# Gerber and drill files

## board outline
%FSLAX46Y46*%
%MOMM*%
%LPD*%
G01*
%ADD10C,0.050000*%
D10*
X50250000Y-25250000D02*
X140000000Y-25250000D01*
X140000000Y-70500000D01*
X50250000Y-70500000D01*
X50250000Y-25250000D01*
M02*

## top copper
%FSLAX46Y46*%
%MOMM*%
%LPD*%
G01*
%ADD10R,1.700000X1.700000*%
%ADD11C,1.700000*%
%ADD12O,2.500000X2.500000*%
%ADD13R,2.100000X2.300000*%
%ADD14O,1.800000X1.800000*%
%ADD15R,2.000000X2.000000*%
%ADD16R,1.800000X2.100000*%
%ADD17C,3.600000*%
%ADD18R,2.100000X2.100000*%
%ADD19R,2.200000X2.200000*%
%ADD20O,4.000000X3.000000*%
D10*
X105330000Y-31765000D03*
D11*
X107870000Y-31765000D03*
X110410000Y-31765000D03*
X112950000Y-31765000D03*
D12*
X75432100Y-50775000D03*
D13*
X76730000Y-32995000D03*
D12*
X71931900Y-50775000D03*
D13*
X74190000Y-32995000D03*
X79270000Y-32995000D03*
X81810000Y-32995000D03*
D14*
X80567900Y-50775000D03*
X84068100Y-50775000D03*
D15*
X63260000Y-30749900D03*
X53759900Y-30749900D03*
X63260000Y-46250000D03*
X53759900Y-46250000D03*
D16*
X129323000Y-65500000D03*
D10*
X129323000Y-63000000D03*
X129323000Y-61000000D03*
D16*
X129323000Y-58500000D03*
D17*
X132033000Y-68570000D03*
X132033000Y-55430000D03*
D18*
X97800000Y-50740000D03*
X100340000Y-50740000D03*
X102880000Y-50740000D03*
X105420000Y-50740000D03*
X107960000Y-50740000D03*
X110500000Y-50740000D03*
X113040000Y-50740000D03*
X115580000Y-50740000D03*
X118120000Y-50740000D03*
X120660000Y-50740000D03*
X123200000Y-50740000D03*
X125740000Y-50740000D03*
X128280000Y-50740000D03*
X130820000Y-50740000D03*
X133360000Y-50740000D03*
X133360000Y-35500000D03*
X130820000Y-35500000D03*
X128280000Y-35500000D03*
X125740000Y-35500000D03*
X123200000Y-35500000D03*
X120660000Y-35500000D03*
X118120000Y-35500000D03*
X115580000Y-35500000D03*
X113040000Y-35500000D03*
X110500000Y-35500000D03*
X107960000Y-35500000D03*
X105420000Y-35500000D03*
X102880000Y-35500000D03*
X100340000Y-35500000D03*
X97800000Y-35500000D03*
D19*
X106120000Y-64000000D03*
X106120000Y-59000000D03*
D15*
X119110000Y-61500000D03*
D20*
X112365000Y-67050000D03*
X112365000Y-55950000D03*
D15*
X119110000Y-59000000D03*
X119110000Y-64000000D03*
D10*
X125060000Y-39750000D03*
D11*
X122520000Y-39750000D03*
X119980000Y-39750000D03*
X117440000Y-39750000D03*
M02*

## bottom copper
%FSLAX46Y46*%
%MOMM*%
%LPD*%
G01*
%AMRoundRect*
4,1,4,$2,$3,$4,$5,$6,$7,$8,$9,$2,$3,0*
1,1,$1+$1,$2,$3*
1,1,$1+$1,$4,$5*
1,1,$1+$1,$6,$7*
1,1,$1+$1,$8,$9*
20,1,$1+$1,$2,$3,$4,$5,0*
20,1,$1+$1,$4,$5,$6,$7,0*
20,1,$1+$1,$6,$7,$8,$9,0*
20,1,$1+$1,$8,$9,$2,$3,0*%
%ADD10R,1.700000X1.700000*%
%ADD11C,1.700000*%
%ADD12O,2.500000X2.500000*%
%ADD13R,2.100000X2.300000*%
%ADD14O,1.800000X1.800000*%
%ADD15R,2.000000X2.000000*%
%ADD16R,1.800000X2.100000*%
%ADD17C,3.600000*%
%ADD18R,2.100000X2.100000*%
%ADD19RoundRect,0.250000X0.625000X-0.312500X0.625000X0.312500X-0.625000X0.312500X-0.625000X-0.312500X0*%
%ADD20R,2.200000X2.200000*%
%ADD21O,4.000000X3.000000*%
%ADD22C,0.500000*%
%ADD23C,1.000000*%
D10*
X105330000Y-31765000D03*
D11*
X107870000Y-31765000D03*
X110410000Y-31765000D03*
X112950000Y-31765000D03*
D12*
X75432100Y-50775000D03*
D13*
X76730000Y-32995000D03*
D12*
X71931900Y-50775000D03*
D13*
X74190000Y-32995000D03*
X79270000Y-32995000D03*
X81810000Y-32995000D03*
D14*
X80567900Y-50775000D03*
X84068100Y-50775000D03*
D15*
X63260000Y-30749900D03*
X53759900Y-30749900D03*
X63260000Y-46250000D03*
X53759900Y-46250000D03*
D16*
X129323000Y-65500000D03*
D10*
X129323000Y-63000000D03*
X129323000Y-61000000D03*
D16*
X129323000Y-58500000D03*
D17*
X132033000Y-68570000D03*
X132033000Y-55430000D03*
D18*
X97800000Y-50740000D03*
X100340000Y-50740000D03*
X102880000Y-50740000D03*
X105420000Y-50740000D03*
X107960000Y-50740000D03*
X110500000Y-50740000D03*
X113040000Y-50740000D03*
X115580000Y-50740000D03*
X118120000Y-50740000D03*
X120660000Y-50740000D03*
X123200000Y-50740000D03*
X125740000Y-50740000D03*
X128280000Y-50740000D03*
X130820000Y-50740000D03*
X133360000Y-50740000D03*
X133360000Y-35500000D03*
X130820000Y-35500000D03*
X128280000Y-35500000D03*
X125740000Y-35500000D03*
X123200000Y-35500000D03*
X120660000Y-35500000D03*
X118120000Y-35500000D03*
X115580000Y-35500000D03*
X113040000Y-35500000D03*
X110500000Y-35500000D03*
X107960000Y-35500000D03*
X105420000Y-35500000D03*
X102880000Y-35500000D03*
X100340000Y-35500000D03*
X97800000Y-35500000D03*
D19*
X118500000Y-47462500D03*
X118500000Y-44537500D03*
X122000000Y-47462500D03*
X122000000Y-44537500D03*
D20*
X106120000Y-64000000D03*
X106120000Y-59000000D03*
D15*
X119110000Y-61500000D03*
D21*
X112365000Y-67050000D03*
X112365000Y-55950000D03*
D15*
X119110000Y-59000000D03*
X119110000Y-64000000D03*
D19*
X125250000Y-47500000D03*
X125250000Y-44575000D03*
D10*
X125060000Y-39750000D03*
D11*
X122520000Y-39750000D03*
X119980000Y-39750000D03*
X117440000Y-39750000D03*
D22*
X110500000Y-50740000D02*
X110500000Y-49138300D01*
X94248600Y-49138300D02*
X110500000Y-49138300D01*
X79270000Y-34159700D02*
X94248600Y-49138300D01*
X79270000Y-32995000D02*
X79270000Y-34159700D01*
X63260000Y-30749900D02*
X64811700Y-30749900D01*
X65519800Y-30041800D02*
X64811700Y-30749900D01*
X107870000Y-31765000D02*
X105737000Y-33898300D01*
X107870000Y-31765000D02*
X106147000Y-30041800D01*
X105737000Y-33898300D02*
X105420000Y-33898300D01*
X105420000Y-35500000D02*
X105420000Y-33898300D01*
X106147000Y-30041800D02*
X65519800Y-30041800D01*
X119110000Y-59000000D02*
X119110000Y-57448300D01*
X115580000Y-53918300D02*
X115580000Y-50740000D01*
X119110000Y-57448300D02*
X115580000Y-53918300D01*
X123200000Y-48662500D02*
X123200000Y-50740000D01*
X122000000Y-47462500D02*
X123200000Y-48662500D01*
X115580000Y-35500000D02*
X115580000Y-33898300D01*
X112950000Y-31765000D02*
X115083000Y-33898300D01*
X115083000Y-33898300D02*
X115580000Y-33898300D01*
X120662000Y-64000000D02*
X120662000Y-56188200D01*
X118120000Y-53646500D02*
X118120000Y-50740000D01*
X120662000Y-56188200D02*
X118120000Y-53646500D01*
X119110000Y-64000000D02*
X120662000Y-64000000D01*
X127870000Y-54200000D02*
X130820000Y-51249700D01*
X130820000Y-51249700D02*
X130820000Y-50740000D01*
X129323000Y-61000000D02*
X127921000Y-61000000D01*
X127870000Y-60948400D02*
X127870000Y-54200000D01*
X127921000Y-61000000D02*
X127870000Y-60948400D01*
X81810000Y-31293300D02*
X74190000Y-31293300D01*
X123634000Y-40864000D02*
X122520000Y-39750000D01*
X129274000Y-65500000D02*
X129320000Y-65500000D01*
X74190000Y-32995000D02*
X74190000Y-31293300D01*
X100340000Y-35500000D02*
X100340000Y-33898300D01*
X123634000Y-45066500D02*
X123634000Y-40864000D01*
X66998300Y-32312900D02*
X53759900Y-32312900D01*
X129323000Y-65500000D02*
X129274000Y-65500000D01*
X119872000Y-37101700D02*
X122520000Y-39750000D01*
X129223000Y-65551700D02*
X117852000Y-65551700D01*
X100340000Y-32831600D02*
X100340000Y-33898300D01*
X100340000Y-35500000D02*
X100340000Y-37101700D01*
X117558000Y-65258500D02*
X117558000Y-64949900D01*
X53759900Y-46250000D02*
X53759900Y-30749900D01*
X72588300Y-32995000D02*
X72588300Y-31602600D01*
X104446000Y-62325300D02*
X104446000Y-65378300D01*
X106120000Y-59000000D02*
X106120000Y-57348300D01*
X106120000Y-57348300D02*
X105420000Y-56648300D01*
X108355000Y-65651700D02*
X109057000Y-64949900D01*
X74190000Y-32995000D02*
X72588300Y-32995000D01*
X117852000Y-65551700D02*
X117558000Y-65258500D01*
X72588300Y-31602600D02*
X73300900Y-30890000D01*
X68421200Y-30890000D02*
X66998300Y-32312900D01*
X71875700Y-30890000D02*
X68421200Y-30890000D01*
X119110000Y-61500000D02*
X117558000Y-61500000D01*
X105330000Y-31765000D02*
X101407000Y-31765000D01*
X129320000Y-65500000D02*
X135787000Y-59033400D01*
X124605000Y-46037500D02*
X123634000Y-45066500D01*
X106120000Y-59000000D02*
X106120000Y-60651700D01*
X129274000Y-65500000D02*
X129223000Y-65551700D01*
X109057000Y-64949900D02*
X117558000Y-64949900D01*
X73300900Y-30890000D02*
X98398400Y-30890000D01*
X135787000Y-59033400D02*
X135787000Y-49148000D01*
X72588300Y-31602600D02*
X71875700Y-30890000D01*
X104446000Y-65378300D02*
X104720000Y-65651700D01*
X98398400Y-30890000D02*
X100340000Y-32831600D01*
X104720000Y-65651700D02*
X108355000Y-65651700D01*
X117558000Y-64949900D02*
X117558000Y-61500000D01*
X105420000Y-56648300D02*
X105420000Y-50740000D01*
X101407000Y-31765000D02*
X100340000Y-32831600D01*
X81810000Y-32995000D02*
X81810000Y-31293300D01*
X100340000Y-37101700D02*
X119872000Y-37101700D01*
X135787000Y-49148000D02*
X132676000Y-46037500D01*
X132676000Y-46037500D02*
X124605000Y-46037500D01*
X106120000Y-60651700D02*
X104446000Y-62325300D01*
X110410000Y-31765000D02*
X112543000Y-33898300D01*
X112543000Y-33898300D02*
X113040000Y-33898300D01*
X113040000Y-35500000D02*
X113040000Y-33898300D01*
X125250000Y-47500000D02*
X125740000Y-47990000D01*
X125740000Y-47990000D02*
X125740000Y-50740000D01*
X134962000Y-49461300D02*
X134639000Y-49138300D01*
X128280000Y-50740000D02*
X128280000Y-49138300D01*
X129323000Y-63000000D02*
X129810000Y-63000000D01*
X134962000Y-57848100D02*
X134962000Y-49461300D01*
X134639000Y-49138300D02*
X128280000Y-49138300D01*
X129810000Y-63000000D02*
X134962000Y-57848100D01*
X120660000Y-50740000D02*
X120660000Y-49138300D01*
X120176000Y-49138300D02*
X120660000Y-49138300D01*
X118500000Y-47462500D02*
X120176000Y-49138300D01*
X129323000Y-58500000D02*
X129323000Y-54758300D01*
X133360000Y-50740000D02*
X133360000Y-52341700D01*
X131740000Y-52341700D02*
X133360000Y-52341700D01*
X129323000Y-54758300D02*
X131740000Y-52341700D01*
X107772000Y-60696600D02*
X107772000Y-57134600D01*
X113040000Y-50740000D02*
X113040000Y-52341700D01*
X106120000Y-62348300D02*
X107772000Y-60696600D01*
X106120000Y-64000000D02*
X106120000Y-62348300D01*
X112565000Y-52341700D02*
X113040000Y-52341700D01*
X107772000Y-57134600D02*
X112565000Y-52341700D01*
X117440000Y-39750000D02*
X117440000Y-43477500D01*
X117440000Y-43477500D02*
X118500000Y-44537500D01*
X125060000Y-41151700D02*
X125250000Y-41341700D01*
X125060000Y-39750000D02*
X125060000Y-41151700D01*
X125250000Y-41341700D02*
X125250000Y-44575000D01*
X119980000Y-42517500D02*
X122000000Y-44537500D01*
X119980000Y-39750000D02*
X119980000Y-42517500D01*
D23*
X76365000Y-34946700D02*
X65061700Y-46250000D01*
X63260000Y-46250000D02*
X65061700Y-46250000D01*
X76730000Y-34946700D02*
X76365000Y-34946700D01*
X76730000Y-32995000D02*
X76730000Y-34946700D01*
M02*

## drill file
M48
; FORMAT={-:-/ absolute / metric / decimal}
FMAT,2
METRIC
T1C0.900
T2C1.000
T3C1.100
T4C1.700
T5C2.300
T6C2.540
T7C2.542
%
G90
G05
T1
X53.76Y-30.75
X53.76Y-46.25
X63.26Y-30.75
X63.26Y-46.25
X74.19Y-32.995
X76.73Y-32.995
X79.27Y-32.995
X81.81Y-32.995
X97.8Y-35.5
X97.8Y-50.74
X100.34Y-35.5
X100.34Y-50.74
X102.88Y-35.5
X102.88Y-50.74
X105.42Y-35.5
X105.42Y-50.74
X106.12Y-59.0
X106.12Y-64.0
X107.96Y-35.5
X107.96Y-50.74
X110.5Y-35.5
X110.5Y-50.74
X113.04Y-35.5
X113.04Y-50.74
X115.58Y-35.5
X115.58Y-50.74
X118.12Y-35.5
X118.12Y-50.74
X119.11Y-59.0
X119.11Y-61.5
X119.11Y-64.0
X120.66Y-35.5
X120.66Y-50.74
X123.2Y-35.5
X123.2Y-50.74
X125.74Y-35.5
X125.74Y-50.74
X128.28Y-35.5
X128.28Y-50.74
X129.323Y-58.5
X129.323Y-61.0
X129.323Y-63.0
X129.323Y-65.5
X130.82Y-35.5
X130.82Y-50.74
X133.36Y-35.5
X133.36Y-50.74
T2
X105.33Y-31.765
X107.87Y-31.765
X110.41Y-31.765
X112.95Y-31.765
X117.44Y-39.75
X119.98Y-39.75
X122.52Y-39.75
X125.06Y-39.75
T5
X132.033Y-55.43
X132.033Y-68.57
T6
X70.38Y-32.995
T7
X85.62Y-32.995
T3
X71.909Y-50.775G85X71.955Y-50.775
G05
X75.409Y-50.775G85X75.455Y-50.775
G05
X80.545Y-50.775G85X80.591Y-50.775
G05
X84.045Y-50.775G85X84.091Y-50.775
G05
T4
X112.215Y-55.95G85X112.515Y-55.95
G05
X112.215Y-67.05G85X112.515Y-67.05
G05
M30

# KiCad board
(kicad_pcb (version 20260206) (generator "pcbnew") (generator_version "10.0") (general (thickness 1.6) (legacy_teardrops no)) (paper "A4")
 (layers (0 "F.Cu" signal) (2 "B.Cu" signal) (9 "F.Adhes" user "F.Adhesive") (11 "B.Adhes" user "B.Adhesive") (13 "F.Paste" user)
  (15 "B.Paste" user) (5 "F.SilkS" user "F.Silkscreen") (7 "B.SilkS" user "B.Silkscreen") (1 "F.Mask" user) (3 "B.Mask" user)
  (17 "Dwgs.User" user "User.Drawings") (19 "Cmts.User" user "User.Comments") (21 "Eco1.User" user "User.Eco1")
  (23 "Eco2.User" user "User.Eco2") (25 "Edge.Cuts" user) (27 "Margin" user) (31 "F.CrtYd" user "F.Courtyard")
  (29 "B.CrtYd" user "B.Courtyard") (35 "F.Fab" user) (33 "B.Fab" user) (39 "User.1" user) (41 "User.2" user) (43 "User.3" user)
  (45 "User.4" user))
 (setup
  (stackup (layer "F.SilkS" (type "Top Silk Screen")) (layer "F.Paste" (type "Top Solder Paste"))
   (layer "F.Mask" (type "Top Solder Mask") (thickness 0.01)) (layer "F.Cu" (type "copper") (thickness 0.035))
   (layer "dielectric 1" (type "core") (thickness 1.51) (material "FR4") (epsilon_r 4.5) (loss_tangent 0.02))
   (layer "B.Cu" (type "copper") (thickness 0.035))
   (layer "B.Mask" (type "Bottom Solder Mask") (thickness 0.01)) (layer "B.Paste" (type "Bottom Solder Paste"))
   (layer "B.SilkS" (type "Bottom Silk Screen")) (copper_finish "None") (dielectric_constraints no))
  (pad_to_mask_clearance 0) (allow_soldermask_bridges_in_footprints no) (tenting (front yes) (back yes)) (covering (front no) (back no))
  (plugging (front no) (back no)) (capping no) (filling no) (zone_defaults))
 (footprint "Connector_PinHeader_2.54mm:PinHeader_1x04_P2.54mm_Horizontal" (layer "F.Cu") (at 105.33 31.765 90)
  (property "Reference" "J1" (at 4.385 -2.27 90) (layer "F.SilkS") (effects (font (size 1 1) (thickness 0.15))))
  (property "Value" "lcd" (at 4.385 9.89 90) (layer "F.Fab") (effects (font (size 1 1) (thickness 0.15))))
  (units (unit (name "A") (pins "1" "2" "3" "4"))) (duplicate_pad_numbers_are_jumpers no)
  (pad "1" thru_hole rect (at 0 0 90) (size 1.7 1.7) (drill 1) (layers "*.Cu" "*.Mask") (remove_unused_layers no) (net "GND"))
  (pad "2" thru_hole circle (at 0 2.54 90) (size 1.7 1.7) (drill 1) (layers "*.Cu" "*.Mask") (remove_unused_layers no) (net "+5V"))
  (pad "3" thru_hole circle (at 0 5.08 90) (size 1.7 1.7) (drill 1) (layers "*.Cu" "*.Mask") (remove_unused_layers no) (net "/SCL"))
  (pad "4" thru_hole circle (at 0 7.62 90) (size 1.7 1.7) (drill 1) (layers "*.Cu" "*.Mask") (remove_unused_layers no) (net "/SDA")))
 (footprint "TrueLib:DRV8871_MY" (layer "F.Cu") (at 78 41.885)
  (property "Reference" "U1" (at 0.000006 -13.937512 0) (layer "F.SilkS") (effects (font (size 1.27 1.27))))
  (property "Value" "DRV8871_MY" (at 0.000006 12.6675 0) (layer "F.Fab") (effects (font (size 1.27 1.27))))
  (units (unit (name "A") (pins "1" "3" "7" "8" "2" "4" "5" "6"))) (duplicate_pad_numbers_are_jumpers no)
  (pad "" np_thru_hole circle (at -7.62 -8.89) (size 2.54 2.54) (drill 2.54) (layers "*.Cu" "*.Mask"))
  (pad "" np_thru_hole circle (at 7.62 -8.89) (size 2.542 2.542) (drill 2.542) (layers "*.Cu" "*.Mask"))
  (pad "1" thru_hole oval (at -2.5679 8.89) (size 2.5 2.5) (drill oval 1.1457 1.1) (layers "*.Cu" "*.Mask") (remove_unused_layers no)
   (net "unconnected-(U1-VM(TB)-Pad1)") (solder_mask_margin 0.1016) (solder_paste_margin 0) (thermal_bridge_angle 0))
  (pad "2" thru_hole rect (at -1.27 -8.89) (size 2.1 2.3) (drill 0.9) (layers "*.Cu" "*.Mask") (remove_unused_layers no) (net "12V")
   (solder_mask_margin 0.102) (solder_paste_margin 0) (thermal_bridge_angle 0))
  (pad "3" thru_hole oval (at -6.0681 8.89) (size 2.5 2.5) (drill oval 1.1457 1.1) (layers "*.Cu" "*.Mask") (remove_unused_layers no)
   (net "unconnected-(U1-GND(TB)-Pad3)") (solder_mask_margin 0.1016) (solder_paste_margin 0) (thermal_bridge_angle 0))
  (pad "4" thru_hole rect (at -3.81 -8.89) (size 2.1 2.3) (drill 0.9) (layers "*.Cu" "*.Mask") (remove_unused_layers no) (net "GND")
   (solder_mask_margin 0.102) (solder_paste_margin 0) (thermal_bridge_angle 0))
  (pad "5" thru_hole rect (at 1.27 -8.89) (size 2.1 2.3) (drill 0.9) (layers "*.Cu" "*.Mask") (remove_unused_layers no) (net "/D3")
   (solder_mask_margin 0.102) (solder_paste_margin 0) (thermal_bridge_angle 0))
  (pad "6" thru_hole rect (at 3.81 -8.89) (size 2.1 2.3) (drill 0.9) (layers "*.Cu" "*.Mask") (remove_unused_layers no) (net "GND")
   (solder_mask_margin 0.102) (solder_paste_margin 0) (thermal_bridge_angle 0))
  (pad "7" thru_hole oval (at 2.5679 8.89) (size 1.8 1.8) (drill oval 1.1457 1.1) (layers "*.Cu" "*.Mask") (remove_unused_layers no)
   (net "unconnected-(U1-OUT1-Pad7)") (solder_mask_margin 0.1016) (solder_paste_margin 0) (thermal_bridge_angle 0))
  (pad "8" thru_hole oval (at 6.0681 8.89) (size 1.8 1.8) (drill oval 1.1457 1.1) (layers "*.Cu" "*.Mask") (remove_unused_layers no)
   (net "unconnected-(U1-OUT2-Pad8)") (solder_mask_margin 0.1016) (solder_paste_margin 0) (thermal_bridge_angle 0)))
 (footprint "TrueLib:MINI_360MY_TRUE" (layer "F.Cu") (at 63.26 46.25 90)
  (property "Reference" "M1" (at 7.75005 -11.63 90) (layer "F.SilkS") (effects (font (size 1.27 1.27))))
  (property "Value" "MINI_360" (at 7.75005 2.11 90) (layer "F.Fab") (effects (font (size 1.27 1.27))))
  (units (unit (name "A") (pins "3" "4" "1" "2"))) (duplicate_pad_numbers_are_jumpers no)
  (pad "1" thru_hole rect (at 15.5001 0 90) (size 2 2) (drill 0.9) (layers "*.Cu" "*.Mask") (remove_unused_layers no) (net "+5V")
   (solder_mask_margin 0.1) (solder_paste_margin 0) (thermal_bridge_angle 0))
  (pad "2" thru_hole rect (at 15.5001 -9.5001 90) (size 2 2) (drill 0.9) (layers "*.Cu" "*.Mask") (remove_unused_layers no) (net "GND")
   (solder_mask_margin 0.1) (solder_paste_margin 0) (thermal_bridge_angle 0))
  (pad "3" thru_hole rect (at 0 0 90) (size 2 2) (drill 0.9) (layers "*.Cu" "*.Mask") (remove_unused_layers no) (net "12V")
   (solder_mask_margin 0.1) (solder_paste_margin 0) (thermal_bridge_angle 0))
  (pad "4" thru_hole rect (at 0 -9.5001 90) (size 2 2) (drill 0.9) (layers "*.Cu" "*.Mask") (remove_unused_layers no) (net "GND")
   (solder_mask_margin 0.1) (solder_paste_margin 0) (thermal_bridge_angle 0)))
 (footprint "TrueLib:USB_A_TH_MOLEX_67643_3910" (layer "F.Cu") (at 129.323 65.5 90)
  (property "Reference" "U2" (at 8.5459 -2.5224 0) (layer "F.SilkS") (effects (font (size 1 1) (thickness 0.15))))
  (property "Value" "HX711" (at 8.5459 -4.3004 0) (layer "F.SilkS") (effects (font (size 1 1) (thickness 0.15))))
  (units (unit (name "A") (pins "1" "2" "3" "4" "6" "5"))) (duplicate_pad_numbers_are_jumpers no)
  (pad "1" thru_hole rect (at 0 0 90) (size 2.1 1.8) (drill 0.9) (layers "*.Cu" "*.Mask") (remove_unused_layers no) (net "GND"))
  (pad "2" thru_hole rect (at 2.5 0 90) (size 1.7 1.7) (drill 0.9) (layers "*.Cu" "*.Mask") (remove_unused_layers no) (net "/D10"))
  (pad "3" thru_hole rect (at 4.5 0 90) (size 1.7 1.7) (drill 0.9) (layers "*.Cu" "*.Mask") (remove_unused_layers no) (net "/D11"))
  (pad "4" thru_hole rect (at 7 0 90) (size 2.1 1.8) (drill 0.9) (layers "*.Cu" "*.Mask") (remove_unused_layers no) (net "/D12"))
  (pad "5" thru_hole circle (at -3.07 2.71 90) (size 3.6 3.6) (drill 2.3) (layers "*.Cu" "*.Mask") (remove_unused_layers no)
   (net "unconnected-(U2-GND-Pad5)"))
  (pad "6" thru_hole circle (at 10.07 2.71 90) (size 3.6 3.6) (drill 2.3) (layers "*.Cu" "*.Mask") (remove_unused_layers no)
   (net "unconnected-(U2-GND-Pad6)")))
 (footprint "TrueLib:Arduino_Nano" (layer "F.Cu") (at 97.8 50.74 90)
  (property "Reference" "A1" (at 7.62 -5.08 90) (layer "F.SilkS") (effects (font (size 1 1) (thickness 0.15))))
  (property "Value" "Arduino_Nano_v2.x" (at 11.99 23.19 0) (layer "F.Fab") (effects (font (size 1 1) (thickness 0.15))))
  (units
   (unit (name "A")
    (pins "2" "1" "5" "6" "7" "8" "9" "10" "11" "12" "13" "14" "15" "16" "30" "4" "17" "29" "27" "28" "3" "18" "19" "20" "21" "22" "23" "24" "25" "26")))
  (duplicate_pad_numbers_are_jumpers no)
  (pad "1" thru_hole rect (at 0 0 90) (size 2.1 2.1) (drill 0.9) (layers "*.Cu" "*.Mask") (remove_unused_layers no)
   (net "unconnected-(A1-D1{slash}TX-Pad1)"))
  (pad "2" thru_hole rect (at 0 2.54 90) (size 2.1 2.1) (drill 0.9) (layers "*.Cu" "*.Mask") (remove_unused_layers no)
   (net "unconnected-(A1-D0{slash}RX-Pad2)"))
  (pad "3" thru_hole rect (at 0 5.08 90) (size 2.1 2.1) (drill 0.9) (layers "*.Cu" "*.Mask") (remove_unused_layers no)
   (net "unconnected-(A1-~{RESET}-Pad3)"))
  (pad "4" thru_hole rect (at 0 7.62 90) (size 2.1 2.1) (drill 0.9) (layers "*.Cu" "*.Mask") (remove_unused_layers no) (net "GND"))
  (pad "5" thru_hole rect (at 0 10.16 90) (size 2.1 2.1) (drill 0.9) (layers "*.Cu" "*.Mask") (remove_unused_layers no)
   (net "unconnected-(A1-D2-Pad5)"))
  (pad "6" thru_hole rect (at 0 12.7 90) (size 2.1 2.1) (drill 0.9) (layers "*.Cu" "*.Mask") (remove_unused_layers no) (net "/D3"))
  (pad "7" thru_hole rect (at 0 15.24 90) (size 2.1 2.1) (drill 0.9) (layers "*.Cu" "*.Mask") (remove_unused_layers no) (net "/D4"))
  (pad "8" thru_hole rect (at 0 17.78 90) (size 2.1 2.1) (drill 0.9) (layers "*.Cu" "*.Mask") (remove_unused_layers no) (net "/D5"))
  (pad "9" thru_hole rect (at 0 20.32 90) (size 2.1 2.1) (drill 0.9) (layers "*.Cu" "*.Mask") (remove_unused_layers no) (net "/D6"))
  (pad "10" thru_hole rect (at 0 22.86 90) (size 2.1 2.1) (drill 0.9) (layers "*.Cu" "*.Mask") (remove_unused_layers no) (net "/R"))
  (pad "11" thru_hole rect (at 0 25.4 90) (size 2.1 2.1) (drill 0.9) (layers "*.Cu" "*.Mask") (remove_unused_layers no) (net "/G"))
  (pad "12" thru_hole rect (at 0 27.94 90) (size 2.1 2.1) (drill 0.9) (layers "*.Cu" "*.Mask") (remove_unused_layers no) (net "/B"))
  (pad "13" thru_hole rect (at 0 30.48 90) (size 2.1 2.1) (drill 0.9) (layers "*.Cu" "*.Mask") (remove_unused_layers no) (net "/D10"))
  (pad "14" thru_hole rect (at 0 33.02 90) (size 2.1 2.1) (drill 0.9) (layers "*.Cu" "*.Mask") (remove_unused_layers no) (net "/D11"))
  (pad "15" thru_hole rect (at 0 35.56 90) (size 2.1 2.1) (drill 0.9) (layers "*.Cu" "*.Mask") (remove_unused_layers no) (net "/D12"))
  (pad "16" thru_hole rect (at 15.24 35.56 90) (size 2.1 2.1) (drill 0.9) (layers "*.Cu" "*.Mask") (remove_unused_layers no)
   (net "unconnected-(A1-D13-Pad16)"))
  (pad "17" thru_hole rect (at 15.24 33.02 90) (size 2.1 2.1) (drill 0.9) (layers "*.Cu" "*.Mask") (remove_unused_layers no)
   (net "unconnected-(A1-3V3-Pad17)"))
  (pad "18" thru_hole rect (at 15.24 30.48 90) (size 2.1 2.1) (drill 0.9) (layers "*.Cu" "*.Mask") (remove_unused_layers no)
   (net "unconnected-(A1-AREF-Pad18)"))
  (pad "19" thru_hole rect (at 15.24 27.94 90) (size 2.1 2.1) (drill 0.9) (layers "*.Cu" "*.Mask") (remove_unused_layers no)
   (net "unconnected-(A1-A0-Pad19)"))
  (pad "20" thru_hole rect (at 15.24 25.4 90) (size 2.1 2.1) (drill 0.9) (layers "*.Cu" "*.Mask") (remove_unused_layers no)
   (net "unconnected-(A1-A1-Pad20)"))
  (pad "21" thru_hole rect (at 15.24 22.86 90) (size 2.1 2.1) (drill 0.9) (layers "*.Cu" "*.Mask") (remove_unused_layers no)
   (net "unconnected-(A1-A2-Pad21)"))
  (pad "22" thru_hole rect (at 15.24 20.32 90) (size 2.1 2.1) (drill 0.9) (layers "*.Cu" "*.Mask") (remove_unused_layers no)
   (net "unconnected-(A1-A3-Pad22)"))
  (pad "23" thru_hole rect (at 15.24 17.78 90) (size 2.1 2.1) (drill 0.9) (layers "*.Cu" "*.Mask") (remove_unused_layers no) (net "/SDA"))
  (pad "24" thru_hole rect (at 15.24 15.24 90) (size 2.1 2.1) (drill 0.9) (layers "*.Cu" "*.Mask") (remove_unused_layers no) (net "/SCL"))
  (pad "25" thru_hole rect (at 15.24 12.7 90) (size 2.1 2.1) (drill 0.9) (layers "*.Cu" "*.Mask") (remove_unused_layers no)
   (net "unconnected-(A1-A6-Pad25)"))
  (pad "26" thru_hole rect (at 15.24 10.16 90) (size 2.1 2.1) (drill 0.9) (layers "*.Cu" "*.Mask") (remove_unused_layers no)
   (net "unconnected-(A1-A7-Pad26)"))
  (pad "27" thru_hole rect (at 15.24 7.62 90) (size 2.1 2.1) (drill 0.9) (layers "*.Cu" "*.Mask") (remove_unused_layers no) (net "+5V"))
  (pad "28" thru_hole rect (at 15.24 5.08 90) (size 2.1 2.1) (drill 0.9) (layers "*.Cu" "*.Mask") (remove_unused_layers no)
   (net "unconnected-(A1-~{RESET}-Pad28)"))
  (pad "29" thru_hole rect (at 15.24 2.54 90) (size 2.1 2.1) (drill 0.9) (layers "*.Cu" "*.Mask") (remove_unused_layers no) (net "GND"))
  (pad "30" thru_hole rect (at 15.24 0 90) (size 2.1 2.1) (drill 0.9) (layers "*.Cu" "*.Mask") (remove_unused_layers no)
   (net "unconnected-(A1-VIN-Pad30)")))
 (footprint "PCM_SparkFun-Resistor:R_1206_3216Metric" (layer "B.Cu") (at 118.5 46 90)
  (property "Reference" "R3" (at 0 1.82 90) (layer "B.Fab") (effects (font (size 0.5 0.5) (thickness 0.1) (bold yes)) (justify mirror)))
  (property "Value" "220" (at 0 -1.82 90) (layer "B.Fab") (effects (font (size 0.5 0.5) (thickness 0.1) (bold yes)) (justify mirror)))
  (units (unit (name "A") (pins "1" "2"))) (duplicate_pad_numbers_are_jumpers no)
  (pad "1" smd roundrect (at -1.4625 0 90) (size 1.125 1.75) (layers "B.Cu" "B.Mask" "B.Paste") (roundrect_rratio 0.222222) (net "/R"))
  (pad "2" smd roundrect (at 1.4625 0 90) (size 1.125 1.75) (layers "B.Cu" "B.Mask" "B.Paste") (roundrect_rratio 0.222222)
   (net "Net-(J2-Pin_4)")))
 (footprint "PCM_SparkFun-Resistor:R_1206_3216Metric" (layer "B.Cu") (at 122 46 90)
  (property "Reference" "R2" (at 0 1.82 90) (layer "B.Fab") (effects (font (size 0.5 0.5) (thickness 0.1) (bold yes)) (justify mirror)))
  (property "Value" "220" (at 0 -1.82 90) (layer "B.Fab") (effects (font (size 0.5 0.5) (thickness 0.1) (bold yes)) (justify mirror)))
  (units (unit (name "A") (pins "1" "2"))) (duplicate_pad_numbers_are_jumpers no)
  (pad "1" smd roundrect (at -1.4625 0 90) (size 1.125 1.75) (layers "B.Cu" "B.Mask" "B.Paste") (roundrect_rratio 0.222222) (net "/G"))
  (pad "2" smd roundrect (at 1.4625 0 90) (size 1.125 1.75) (layers "B.Cu" "B.Mask" "B.Paste") (roundrect_rratio 0.222222)
   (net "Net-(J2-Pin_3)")))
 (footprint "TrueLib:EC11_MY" (layer "B.Cu") (at 112.115 61.5 90)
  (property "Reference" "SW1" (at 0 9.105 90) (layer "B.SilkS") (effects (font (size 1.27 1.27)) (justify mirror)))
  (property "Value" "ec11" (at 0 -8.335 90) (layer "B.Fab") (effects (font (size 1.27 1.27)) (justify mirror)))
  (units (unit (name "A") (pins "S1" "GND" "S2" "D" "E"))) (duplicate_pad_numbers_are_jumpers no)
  (pad "D" thru_hole rect (at -2.5 -5.995 90) (size 2.2 2.2) (drill 0.9) (layers "*.Cu" "*.Mask") (remove_unused_layers no) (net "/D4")
   (solder_mask_margin 0.05) (solder_paste_margin 0) (thermal_bridge_angle 0))
  (pad "E" thru_hole rect (at 2.5 -5.995 90) (size 2.2 2.2) (drill 0.9) (layers "*.Cu" "*.Mask") (remove_unused_layers no) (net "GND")
   (solder_mask_margin 0.05) (solder_paste_margin 0) (thermal_bridge_angle 0))
  (pad "GND" thru_hole rect (at 0 6.995 90) (size 2 2) (drill 0.9) (layers "*.Cu" "*.Mask") (remove_unused_layers no) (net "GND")
   (solder_mask_margin 0.05) (solder_paste_margin 0) (thermal_bridge_angle 0))
  (pad "MP1" thru_hole oval (at -5.55 0.25 90) (size 3 4) (drill oval 1.7 2) (layers "*.Cu" "*.Mask") (remove_unused_layers no)
   (solder_mask_margin 0.05) (solder_paste_margin 0) (thermal_bridge_angle 0))
  (pad "MP2" thru_hole oval (at 5.55 0.25 90) (size 3 4) (drill oval 1.7 2) (layers "*.Cu" "*.Mask") (remove_unused_layers no)
   (solder_mask_margin 0.05) (solder_paste_margin 0) (thermal_bridge_angle 0))
  (pad "S1" thru_hole rect (at 2.5 6.995 90) (size 2 2) (drill 0.9) (layers "*.Cu" "*.Mask") (remove_unused_layers no) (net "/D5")
   (solder_mask_margin 0.05) (solder_paste_margin 0) (thermal_bridge_angle 0))
  (pad "S2" thru_hole rect (at -2.5 6.995 90) (size 2 2) (drill 0.9) (layers "*.Cu" "*.Mask") (remove_unused_layers no) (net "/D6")
   (solder_mask_margin 0.05) (solder_paste_margin 0) (thermal_bridge_angle 0))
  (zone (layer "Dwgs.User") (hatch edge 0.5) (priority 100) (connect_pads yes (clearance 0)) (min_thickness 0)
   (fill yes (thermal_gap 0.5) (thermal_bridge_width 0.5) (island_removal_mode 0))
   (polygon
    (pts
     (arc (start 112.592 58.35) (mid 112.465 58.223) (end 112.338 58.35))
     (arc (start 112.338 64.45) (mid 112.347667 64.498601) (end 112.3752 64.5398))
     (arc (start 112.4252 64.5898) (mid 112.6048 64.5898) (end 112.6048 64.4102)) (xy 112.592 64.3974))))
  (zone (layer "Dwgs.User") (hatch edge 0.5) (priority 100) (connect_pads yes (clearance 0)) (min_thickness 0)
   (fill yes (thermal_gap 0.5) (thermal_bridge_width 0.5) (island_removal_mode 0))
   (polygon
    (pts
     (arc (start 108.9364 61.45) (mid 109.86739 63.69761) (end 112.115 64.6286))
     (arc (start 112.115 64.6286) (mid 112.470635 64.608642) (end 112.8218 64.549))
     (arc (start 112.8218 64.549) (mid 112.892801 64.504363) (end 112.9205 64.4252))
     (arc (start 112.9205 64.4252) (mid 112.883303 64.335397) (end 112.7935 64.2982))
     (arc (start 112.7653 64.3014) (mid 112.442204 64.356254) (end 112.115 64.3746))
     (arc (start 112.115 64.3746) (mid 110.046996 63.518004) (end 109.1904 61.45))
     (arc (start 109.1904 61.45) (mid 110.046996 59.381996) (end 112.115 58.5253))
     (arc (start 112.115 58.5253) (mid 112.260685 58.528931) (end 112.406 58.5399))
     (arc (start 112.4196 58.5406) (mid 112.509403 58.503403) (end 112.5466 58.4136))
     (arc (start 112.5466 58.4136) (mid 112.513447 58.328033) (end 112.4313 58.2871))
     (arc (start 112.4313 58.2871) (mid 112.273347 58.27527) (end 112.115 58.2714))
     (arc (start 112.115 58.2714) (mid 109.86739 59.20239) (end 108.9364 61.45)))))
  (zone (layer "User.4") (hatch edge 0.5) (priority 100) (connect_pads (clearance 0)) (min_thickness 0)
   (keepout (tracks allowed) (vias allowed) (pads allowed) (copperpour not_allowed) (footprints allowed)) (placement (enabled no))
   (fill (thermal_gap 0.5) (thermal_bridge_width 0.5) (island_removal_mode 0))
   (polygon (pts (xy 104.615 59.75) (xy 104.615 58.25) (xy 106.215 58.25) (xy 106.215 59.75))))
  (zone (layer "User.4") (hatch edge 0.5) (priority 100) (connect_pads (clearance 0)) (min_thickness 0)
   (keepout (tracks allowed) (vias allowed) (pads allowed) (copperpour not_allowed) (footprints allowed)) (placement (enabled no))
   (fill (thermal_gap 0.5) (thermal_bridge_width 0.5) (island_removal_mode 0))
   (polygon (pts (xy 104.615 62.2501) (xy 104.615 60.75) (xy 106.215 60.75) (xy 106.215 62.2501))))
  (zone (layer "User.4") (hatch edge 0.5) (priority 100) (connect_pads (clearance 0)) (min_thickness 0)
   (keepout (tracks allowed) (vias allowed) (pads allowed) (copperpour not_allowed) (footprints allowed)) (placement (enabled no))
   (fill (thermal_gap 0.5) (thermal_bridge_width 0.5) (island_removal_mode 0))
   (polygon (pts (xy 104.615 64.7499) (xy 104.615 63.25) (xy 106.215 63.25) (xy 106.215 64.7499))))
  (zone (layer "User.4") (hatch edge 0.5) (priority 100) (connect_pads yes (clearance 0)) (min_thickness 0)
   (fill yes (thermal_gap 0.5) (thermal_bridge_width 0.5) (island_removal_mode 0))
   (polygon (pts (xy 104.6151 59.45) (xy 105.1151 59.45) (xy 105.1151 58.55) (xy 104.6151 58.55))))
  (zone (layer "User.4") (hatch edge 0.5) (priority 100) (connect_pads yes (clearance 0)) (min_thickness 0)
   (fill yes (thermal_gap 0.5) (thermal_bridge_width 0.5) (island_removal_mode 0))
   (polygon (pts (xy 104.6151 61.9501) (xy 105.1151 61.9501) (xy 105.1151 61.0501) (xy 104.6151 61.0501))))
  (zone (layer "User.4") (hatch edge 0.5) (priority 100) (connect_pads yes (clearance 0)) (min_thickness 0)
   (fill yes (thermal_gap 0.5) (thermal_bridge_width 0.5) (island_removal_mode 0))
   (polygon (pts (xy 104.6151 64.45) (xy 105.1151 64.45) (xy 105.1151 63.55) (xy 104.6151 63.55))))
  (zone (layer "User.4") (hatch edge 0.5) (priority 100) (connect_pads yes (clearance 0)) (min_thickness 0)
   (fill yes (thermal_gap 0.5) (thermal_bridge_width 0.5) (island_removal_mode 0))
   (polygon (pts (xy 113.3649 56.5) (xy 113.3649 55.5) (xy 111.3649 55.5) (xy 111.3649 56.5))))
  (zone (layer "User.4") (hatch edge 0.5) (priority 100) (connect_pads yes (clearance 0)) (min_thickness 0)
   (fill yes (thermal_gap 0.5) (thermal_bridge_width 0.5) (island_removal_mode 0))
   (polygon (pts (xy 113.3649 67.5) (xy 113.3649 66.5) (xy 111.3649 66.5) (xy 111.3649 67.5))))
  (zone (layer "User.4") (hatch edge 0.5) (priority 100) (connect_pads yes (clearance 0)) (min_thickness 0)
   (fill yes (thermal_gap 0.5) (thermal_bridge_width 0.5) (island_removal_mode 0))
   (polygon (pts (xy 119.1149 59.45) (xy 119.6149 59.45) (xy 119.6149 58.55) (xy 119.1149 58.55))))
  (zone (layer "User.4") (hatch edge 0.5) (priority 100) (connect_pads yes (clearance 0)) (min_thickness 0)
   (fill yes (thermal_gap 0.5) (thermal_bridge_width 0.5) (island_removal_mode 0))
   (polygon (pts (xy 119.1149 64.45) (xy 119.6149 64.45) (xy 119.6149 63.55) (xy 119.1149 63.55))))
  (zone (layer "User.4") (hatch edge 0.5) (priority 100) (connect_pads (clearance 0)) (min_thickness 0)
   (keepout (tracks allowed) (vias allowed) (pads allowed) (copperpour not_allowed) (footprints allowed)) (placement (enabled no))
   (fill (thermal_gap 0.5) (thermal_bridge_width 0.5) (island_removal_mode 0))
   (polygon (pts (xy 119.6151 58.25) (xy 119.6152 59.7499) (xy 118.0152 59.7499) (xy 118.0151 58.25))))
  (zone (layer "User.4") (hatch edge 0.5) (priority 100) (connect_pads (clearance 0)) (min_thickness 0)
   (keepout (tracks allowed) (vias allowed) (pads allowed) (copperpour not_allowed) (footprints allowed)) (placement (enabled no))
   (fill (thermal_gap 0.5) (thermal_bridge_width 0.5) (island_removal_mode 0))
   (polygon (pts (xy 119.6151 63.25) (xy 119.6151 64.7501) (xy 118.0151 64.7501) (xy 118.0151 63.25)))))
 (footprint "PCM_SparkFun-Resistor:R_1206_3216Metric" (layer "B.Cu") (at 125.25 46.0375 90)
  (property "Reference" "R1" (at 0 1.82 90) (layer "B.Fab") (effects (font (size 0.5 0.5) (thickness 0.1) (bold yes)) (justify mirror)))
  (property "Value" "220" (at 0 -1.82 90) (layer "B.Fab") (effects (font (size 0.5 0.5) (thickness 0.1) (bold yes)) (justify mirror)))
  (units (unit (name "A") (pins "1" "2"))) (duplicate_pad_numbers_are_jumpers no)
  (pad "1" smd roundrect (at -1.4625 0 90) (size 1.125 1.75) (layers "B.Cu" "B.Mask" "B.Paste") (roundrect_rratio 0.222222) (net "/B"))
  (pad "2" smd roundrect (at 1.4625 0 90) (size 1.125 1.75) (layers "B.Cu" "B.Mask" "B.Paste") (roundrect_rratio 0.222222)
   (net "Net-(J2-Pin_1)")))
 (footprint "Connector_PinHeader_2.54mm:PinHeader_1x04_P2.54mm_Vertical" (layer "B.Cu") (at 125.06 39.75 90)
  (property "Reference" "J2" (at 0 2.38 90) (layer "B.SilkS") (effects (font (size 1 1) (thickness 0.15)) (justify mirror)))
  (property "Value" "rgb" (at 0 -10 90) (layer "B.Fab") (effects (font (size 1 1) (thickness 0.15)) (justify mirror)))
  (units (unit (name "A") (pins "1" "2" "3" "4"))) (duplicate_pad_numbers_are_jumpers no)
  (pad "1" thru_hole rect (at 0 0 90) (size 1.7 1.7) (drill 1) (layers "*.Cu" "*.Mask") (remove_unused_layers no) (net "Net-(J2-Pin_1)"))
  (pad "2" thru_hole circle (at 0 -2.54 90) (size 1.7 1.7) (drill 1) (layers "*.Cu" "*.Mask") (remove_unused_layers no) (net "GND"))
  (pad "3" thru_hole circle (at 0 -5.08 90) (size 1.7 1.7) (drill 1) (layers "*.Cu" "*.Mask") (remove_unused_layers no)
   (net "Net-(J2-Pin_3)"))
  (pad "4" thru_hole circle (at 0 -7.62 90) (size 1.7 1.7) (drill 1) (layers "*.Cu" "*.Mask") (remove_unused_layers no)
   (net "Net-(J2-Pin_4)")))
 (gr_rect (start 50.25 25.25) (end 140 70.5) (stroke (width 0.05) (type default)) (fill no) (layer "Edge.Cuts"))
 (segment (start 110.5 50.74) (end 110.5 49.1383) (width 0.5) (layer "B.Cu") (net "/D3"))
 (segment (start 94.2486 49.1383) (end 110.5 49.1383) (width 0.5) (layer "B.Cu") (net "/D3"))
 (segment (start 79.27 34.1597) (end 94.2486 49.1383) (width 0.5) (layer "B.Cu") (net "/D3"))
 (segment (start 79.27 32.995) (end 79.27 34.1597) (width 0.5) (layer "B.Cu") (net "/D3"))
 (segment (start 63.26 30.7499) (end 64.8117 30.7499) (width 0.5) (layer "B.Cu") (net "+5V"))
 (segment (start 65.5198 30.0418) (end 64.8117 30.7499) (width 0.5) (layer "B.Cu") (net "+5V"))
 (segment (start 107.87 31.765) (end 105.737 33.8983) (width 0.5) (layer "B.Cu") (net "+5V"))
 (segment (start 107.87 31.765) (end 106.147 30.0418) (width 0.5) (layer "B.Cu") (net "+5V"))
 (segment (start 105.737 33.8983) (end 105.42 33.8983) (width 0.5) (layer "B.Cu") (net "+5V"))
 (segment (start 105.42 35.5) (end 105.42 33.8983) (width 0.5) (layer "B.Cu") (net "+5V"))
 (segment (start 106.147 30.0418) (end 65.5198 30.0418) (width 0.5) (layer "B.Cu") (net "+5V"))
 (segment (start 119.11 59) (end 119.11 57.4483) (width 0.5) (layer "B.Cu") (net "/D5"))
 (segment (start 115.58 53.9183) (end 115.58 50.74) (width 0.5) (layer "B.Cu") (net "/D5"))
 (segment (start 119.11 57.4483) (end 115.58 53.9183) (width 0.5) (layer "B.Cu") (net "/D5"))
 (segment (start 123.2 48.6625) (end 123.2 50.74) (width 0.5) (layer "B.Cu") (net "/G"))
 (segment (start 122 47.4625) (end 123.2 48.6625) (width 0.5) (layer "B.Cu") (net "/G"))
 (segment (start 115.58 35.5) (end 115.58 33.8983) (width 0.5) (layer "B.Cu") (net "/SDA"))
 (segment (start 112.95 31.765) (end 115.083 33.8983) (width 0.5) (layer "B.Cu") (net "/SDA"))
 (segment (start 115.083 33.8983) (end 115.58 33.8983) (width 0.5) (layer "B.Cu") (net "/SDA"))
 (segment (start 120.662 64) (end 120.662 56.1882) (width 0.5) (layer "B.Cu") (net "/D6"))
 (segment (start 118.12 53.6465) (end 118.12 50.74) (width 0.5) (layer "B.Cu") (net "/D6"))
 (segment (start 120.662 56.1882) (end 118.12 53.6465) (width 0.5) (layer "B.Cu") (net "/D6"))
 (segment (start 119.11 64) (end 120.662 64) (width 0.5) (layer "B.Cu") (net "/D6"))
 (segment (start 127.87 54.2) (end 130.82 51.2497) (width 0.5) (layer "B.Cu") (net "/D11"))
 (segment (start 130.82 51.2497) (end 130.82 50.74) (width 0.5) (layer "B.Cu") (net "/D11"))
 (segment (start 129.323 61) (end 127.921 61) (width 0.5) (layer "B.Cu") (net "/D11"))
 (segment (start 127.87 60.9484) (end 127.87 54.2) (width 0.5) (layer "B.Cu") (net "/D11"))
 (segment (start 127.921 61) (end 127.87 60.9484) (width 0.5) (layer "B.Cu") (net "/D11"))
 (segment (start 81.81 31.2933) (end 74.19 31.2933) (width 0.5) (layer "B.Cu") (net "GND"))
 (segment (start 123.634 40.864) (end 122.52 39.75) (width 0.5) (layer "B.Cu") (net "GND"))
 (segment (start 129.274 65.5) (end 129.32 65.5) (width 0.5) (layer "B.Cu") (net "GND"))
 (segment (start 74.19 32.995) (end 74.19 31.2933) (width 0.5) (layer "B.Cu") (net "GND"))
 (segment (start 100.34 35.5) (end 100.34 33.8983) (width 0.5) (layer "B.Cu") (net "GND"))
 (segment (start 123.634 45.0665) (end 123.634 40.864) (width 0.5) (layer "B.Cu") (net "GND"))
 (segment (start 66.9983 32.3129) (end 53.7599 32.3129) (width 0.5) (layer "B.Cu") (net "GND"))
 (segment (start 129.323 65.5) (end 129.274 65.5) (width 0.5) (layer "B.Cu") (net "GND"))
 (segment (start 119.872 37.1017) (end 122.52 39.75) (width 0.5) (layer "B.Cu") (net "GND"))
 (segment (start 129.223 65.5517) (end 117.852 65.5517) (width 0.5) (layer "B.Cu") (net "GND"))
 (segment (start 100.34 32.8316) (end 100.34 33.8983) (width 0.5) (layer "B.Cu") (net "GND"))
 (segment (start 100.34 35.5) (end 100.34 37.1017) (width 0.5) (layer "B.Cu") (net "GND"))
 (segment (start 117.558 65.2585) (end 117.558 64.9499) (width 0.5) (layer "B.Cu") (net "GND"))
 (segment (start 53.7599 46.25) (end 53.7599 30.7499) (width 0.5) (layer "B.Cu") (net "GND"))
 (segment (start 72.5883 32.995) (end 72.5883 31.6026) (width 0.5) (layer "B.Cu") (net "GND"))
 (segment (start 104.446 62.3253) (end 104.446 65.3783) (width 0.5) (layer "B.Cu") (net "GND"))
 (segment (start 106.12 59) (end 106.12 57.3483) (width 0.5) (layer "B.Cu") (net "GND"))
 (segment (start 106.12 57.3483) (end 105.42 56.6483) (width 0.5) (layer "B.Cu") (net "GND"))
 (segment (start 108.355 65.6517) (end 109.057 64.9499) (width 0.5) (layer "B.Cu") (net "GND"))
 (segment (start 74.19 32.995) (end 72.5883 32.995) (width 0.5) (layer "B.Cu") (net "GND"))
 (segment (start 117.852 65.5517) (end 117.558 65.2585) (width 0.5) (layer "B.Cu") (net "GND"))
 (segment (start 72.5883 31.6026) (end 73.3009 30.89) (width 0.5) (layer "B.Cu") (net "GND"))
 (segment (start 68.4212 30.89) (end 66.9983 32.3129) (width 0.5) (layer "B.Cu") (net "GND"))
 (segment (start 71.8757 30.89) (end 68.4212 30.89) (width 0.5) (layer "B.Cu") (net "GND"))
 (segment (start 119.11 61.5) (end 117.558 61.5) (width 0.5) (layer "B.Cu") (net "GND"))
 (segment (start 105.33 31.765) (end 101.407 31.765) (width 0.5) (layer "B.Cu") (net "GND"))
 (segment (start 129.32 65.5) (end 135.787 59.0334) (width 0.5) (layer "B.Cu") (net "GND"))
 (segment (start 124.605 46.0375) (end 123.634 45.0665) (width 0.5) (layer "B.Cu") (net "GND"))
 (segment (start 106.12 59) (end 106.12 60.6517) (width 0.5) (layer "B.Cu") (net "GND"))
 (segment (start 129.274 65.5) (end 129.223 65.5517) (width 0.5) (layer "B.Cu") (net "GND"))
 (segment (start 109.057 64.9499) (end 117.558 64.9499) (width 0.5) (layer "B.Cu") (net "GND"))
 (segment (start 73.3009 30.89) (end 98.3984 30.89) (width 0.5) (layer "B.Cu") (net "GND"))
 (segment (start 135.787 59.0334) (end 135.787 49.148) (width 0.5) (layer "B.Cu") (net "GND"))
 (segment (start 72.5883 31.6026) (end 71.8757 30.89) (width 0.5) (layer "B.Cu") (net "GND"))
 (segment (start 104.446 65.3783) (end 104.72 65.6517) (width 0.5) (layer "B.Cu") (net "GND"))
 (segment (start 98.3984 30.89) (end 100.34 32.8316) (width 0.5) (layer "B.Cu") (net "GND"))
 (segment (start 104.72 65.6517) (end 108.355 65.6517) (width 0.5) (layer "B.Cu") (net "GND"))
 (segment (start 117.558 64.9499) (end 117.558 61.5) (width 0.5) (layer "B.Cu") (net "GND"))
 (segment (start 105.42 56.6483) (end 105.42 50.74) (width 0.5) (layer "B.Cu") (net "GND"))
 (segment (start 101.407 31.765) (end 100.34 32.8316) (width 0.5) (layer "B.Cu") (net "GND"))
 (segment (start 81.81 32.995) (end 81.81 31.2933) (width 0.5) (layer "B.Cu") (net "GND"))
 (segment (start 100.34 37.1017) (end 119.872 37.1017) (width 0.5) (layer "B.Cu") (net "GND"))
 (segment (start 135.787 49.148) (end 132.676 46.0375) (width 0.5) (layer "B.Cu") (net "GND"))
 (segment (start 132.676 46.0375) (end 124.605 46.0375) (width 0.5) (layer "B.Cu") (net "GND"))
 (segment (start 106.12 60.6517) (end 104.446 62.3253) (width 0.5) (layer "B.Cu") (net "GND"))
 (segment (start 110.41 31.765) (end 112.543 33.8983) (width 0.5) (layer "B.Cu") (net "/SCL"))
 (segment (start 112.543 33.8983) (end 113.04 33.8983) (width 0.5) (layer "B.Cu") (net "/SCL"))
 (segment (start 113.04 35.5) (end 113.04 33.8983) (width 0.5) (layer "B.Cu") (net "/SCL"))
 (segment (start 125.25 47.5) (end 125.74 47.99) (width 0.5) (layer "B.Cu") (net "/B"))
 (segment (start 125.74 47.99) (end 125.74 50.74) (width 0.5) (layer "B.Cu") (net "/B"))
 (segment (start 134.962 49.4613) (end 134.639 49.1383) (width 0.5) (layer "B.Cu") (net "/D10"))
 (segment (start 128.28 50.74) (end 128.28 49.1383) (width 0.5) (layer "B.Cu") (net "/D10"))
 (segment (start 129.323 63) (end 129.81 63) (width 0.5) (layer "B.Cu") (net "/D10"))
 (segment (start 134.962 57.8481) (end 134.962 49.4613) (width 0.5) (layer "B.Cu") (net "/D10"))
 (segment (start 134.639 49.1383) (end 128.28 49.1383) (width 0.5) (layer "B.Cu") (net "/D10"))
 (segment (start 129.81 63) (end 134.962 57.8481) (width 0.5) (layer "B.Cu") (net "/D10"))
 (segment (start 120.66 50.74) (end 120.66 49.1383) (width 0.5) (layer "B.Cu") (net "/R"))
 (segment (start 120.176 49.1383) (end 120.66 49.1383) (width 0.5) (layer "B.Cu") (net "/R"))
 (segment (start 118.5 47.4625) (end 120.176 49.1383) (width 0.5) (layer "B.Cu") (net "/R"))
 (segment (start 129.323 58.5) (end 129.323 54.7583) (width 0.5) (layer "B.Cu") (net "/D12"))
 (segment (start 133.36 50.74) (end 133.36 52.3417) (width 0.5) (layer "B.Cu") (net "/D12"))
 (segment (start 131.74 52.3417) (end 133.36 52.3417) (width 0.5) (layer "B.Cu") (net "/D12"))
 (segment (start 129.323 54.7583) (end 131.74 52.3417) (width 0.5) (layer "B.Cu") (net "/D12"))
 (segment (start 107.772 60.6966) (end 107.772 57.1346) (width 0.5) (layer "B.Cu") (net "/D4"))
 (segment (start 113.04 50.74) (end 113.04 52.3417) (width 0.5) (layer "B.Cu") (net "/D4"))
 (segment (start 106.12 62.3483) (end 107.772 60.6966) (width 0.5) (layer "B.Cu") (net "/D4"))
 (segment (start 106.12 64) (end 106.12 62.3483) (width 0.5) (layer "B.Cu") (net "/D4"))
 (segment (start 112.565 52.3417) (end 113.04 52.3417) (width 0.5) (layer "B.Cu") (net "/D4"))
 (segment (start 107.772 57.1346) (end 112.565 52.3417) (width 0.5) (layer "B.Cu") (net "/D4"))
 (segment (start 117.44 39.75) (end 117.44 43.4775) (width 0.5) (layer "B.Cu") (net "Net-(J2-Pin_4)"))
 (segment (start 117.44 43.4775) (end 118.5 44.5375) (width 0.5) (layer "B.Cu") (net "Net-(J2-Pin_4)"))
 (segment (start 125.06 41.1517) (end 125.25 41.3417) (width 0.5) (layer "B.Cu") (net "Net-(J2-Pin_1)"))
 (segment (start 125.06 39.75) (end 125.06 41.1517) (width 0.5) (layer "B.Cu") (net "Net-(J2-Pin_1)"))
 (segment (start 125.25 41.3417) (end 125.25 44.575) (width 0.5) (layer "B.Cu") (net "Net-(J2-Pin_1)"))
 (segment (start 119.98 42.5175) (end 122 44.5375) (width 0.5) (layer "B.Cu") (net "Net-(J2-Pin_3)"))
 (segment (start 119.98 39.75) (end 119.98 42.5175) (width 0.5) (layer "B.Cu") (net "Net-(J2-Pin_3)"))
 (segment (start 76.365 34.9467) (end 65.0617 46.25) (width 1) (layer "B.Cu") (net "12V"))
 (segment (start 63.26 46.25) (end 65.0617 46.25) (width 1) (layer "B.Cu") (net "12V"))
 (segment (start 76.73 34.9467) (end 76.365 34.9467) (width 1) (layer "B.Cu") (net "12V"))
 (segment (start 76.73 32.995) (end 76.73 34.9467) (width 1) (layer "B.Cu") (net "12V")))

